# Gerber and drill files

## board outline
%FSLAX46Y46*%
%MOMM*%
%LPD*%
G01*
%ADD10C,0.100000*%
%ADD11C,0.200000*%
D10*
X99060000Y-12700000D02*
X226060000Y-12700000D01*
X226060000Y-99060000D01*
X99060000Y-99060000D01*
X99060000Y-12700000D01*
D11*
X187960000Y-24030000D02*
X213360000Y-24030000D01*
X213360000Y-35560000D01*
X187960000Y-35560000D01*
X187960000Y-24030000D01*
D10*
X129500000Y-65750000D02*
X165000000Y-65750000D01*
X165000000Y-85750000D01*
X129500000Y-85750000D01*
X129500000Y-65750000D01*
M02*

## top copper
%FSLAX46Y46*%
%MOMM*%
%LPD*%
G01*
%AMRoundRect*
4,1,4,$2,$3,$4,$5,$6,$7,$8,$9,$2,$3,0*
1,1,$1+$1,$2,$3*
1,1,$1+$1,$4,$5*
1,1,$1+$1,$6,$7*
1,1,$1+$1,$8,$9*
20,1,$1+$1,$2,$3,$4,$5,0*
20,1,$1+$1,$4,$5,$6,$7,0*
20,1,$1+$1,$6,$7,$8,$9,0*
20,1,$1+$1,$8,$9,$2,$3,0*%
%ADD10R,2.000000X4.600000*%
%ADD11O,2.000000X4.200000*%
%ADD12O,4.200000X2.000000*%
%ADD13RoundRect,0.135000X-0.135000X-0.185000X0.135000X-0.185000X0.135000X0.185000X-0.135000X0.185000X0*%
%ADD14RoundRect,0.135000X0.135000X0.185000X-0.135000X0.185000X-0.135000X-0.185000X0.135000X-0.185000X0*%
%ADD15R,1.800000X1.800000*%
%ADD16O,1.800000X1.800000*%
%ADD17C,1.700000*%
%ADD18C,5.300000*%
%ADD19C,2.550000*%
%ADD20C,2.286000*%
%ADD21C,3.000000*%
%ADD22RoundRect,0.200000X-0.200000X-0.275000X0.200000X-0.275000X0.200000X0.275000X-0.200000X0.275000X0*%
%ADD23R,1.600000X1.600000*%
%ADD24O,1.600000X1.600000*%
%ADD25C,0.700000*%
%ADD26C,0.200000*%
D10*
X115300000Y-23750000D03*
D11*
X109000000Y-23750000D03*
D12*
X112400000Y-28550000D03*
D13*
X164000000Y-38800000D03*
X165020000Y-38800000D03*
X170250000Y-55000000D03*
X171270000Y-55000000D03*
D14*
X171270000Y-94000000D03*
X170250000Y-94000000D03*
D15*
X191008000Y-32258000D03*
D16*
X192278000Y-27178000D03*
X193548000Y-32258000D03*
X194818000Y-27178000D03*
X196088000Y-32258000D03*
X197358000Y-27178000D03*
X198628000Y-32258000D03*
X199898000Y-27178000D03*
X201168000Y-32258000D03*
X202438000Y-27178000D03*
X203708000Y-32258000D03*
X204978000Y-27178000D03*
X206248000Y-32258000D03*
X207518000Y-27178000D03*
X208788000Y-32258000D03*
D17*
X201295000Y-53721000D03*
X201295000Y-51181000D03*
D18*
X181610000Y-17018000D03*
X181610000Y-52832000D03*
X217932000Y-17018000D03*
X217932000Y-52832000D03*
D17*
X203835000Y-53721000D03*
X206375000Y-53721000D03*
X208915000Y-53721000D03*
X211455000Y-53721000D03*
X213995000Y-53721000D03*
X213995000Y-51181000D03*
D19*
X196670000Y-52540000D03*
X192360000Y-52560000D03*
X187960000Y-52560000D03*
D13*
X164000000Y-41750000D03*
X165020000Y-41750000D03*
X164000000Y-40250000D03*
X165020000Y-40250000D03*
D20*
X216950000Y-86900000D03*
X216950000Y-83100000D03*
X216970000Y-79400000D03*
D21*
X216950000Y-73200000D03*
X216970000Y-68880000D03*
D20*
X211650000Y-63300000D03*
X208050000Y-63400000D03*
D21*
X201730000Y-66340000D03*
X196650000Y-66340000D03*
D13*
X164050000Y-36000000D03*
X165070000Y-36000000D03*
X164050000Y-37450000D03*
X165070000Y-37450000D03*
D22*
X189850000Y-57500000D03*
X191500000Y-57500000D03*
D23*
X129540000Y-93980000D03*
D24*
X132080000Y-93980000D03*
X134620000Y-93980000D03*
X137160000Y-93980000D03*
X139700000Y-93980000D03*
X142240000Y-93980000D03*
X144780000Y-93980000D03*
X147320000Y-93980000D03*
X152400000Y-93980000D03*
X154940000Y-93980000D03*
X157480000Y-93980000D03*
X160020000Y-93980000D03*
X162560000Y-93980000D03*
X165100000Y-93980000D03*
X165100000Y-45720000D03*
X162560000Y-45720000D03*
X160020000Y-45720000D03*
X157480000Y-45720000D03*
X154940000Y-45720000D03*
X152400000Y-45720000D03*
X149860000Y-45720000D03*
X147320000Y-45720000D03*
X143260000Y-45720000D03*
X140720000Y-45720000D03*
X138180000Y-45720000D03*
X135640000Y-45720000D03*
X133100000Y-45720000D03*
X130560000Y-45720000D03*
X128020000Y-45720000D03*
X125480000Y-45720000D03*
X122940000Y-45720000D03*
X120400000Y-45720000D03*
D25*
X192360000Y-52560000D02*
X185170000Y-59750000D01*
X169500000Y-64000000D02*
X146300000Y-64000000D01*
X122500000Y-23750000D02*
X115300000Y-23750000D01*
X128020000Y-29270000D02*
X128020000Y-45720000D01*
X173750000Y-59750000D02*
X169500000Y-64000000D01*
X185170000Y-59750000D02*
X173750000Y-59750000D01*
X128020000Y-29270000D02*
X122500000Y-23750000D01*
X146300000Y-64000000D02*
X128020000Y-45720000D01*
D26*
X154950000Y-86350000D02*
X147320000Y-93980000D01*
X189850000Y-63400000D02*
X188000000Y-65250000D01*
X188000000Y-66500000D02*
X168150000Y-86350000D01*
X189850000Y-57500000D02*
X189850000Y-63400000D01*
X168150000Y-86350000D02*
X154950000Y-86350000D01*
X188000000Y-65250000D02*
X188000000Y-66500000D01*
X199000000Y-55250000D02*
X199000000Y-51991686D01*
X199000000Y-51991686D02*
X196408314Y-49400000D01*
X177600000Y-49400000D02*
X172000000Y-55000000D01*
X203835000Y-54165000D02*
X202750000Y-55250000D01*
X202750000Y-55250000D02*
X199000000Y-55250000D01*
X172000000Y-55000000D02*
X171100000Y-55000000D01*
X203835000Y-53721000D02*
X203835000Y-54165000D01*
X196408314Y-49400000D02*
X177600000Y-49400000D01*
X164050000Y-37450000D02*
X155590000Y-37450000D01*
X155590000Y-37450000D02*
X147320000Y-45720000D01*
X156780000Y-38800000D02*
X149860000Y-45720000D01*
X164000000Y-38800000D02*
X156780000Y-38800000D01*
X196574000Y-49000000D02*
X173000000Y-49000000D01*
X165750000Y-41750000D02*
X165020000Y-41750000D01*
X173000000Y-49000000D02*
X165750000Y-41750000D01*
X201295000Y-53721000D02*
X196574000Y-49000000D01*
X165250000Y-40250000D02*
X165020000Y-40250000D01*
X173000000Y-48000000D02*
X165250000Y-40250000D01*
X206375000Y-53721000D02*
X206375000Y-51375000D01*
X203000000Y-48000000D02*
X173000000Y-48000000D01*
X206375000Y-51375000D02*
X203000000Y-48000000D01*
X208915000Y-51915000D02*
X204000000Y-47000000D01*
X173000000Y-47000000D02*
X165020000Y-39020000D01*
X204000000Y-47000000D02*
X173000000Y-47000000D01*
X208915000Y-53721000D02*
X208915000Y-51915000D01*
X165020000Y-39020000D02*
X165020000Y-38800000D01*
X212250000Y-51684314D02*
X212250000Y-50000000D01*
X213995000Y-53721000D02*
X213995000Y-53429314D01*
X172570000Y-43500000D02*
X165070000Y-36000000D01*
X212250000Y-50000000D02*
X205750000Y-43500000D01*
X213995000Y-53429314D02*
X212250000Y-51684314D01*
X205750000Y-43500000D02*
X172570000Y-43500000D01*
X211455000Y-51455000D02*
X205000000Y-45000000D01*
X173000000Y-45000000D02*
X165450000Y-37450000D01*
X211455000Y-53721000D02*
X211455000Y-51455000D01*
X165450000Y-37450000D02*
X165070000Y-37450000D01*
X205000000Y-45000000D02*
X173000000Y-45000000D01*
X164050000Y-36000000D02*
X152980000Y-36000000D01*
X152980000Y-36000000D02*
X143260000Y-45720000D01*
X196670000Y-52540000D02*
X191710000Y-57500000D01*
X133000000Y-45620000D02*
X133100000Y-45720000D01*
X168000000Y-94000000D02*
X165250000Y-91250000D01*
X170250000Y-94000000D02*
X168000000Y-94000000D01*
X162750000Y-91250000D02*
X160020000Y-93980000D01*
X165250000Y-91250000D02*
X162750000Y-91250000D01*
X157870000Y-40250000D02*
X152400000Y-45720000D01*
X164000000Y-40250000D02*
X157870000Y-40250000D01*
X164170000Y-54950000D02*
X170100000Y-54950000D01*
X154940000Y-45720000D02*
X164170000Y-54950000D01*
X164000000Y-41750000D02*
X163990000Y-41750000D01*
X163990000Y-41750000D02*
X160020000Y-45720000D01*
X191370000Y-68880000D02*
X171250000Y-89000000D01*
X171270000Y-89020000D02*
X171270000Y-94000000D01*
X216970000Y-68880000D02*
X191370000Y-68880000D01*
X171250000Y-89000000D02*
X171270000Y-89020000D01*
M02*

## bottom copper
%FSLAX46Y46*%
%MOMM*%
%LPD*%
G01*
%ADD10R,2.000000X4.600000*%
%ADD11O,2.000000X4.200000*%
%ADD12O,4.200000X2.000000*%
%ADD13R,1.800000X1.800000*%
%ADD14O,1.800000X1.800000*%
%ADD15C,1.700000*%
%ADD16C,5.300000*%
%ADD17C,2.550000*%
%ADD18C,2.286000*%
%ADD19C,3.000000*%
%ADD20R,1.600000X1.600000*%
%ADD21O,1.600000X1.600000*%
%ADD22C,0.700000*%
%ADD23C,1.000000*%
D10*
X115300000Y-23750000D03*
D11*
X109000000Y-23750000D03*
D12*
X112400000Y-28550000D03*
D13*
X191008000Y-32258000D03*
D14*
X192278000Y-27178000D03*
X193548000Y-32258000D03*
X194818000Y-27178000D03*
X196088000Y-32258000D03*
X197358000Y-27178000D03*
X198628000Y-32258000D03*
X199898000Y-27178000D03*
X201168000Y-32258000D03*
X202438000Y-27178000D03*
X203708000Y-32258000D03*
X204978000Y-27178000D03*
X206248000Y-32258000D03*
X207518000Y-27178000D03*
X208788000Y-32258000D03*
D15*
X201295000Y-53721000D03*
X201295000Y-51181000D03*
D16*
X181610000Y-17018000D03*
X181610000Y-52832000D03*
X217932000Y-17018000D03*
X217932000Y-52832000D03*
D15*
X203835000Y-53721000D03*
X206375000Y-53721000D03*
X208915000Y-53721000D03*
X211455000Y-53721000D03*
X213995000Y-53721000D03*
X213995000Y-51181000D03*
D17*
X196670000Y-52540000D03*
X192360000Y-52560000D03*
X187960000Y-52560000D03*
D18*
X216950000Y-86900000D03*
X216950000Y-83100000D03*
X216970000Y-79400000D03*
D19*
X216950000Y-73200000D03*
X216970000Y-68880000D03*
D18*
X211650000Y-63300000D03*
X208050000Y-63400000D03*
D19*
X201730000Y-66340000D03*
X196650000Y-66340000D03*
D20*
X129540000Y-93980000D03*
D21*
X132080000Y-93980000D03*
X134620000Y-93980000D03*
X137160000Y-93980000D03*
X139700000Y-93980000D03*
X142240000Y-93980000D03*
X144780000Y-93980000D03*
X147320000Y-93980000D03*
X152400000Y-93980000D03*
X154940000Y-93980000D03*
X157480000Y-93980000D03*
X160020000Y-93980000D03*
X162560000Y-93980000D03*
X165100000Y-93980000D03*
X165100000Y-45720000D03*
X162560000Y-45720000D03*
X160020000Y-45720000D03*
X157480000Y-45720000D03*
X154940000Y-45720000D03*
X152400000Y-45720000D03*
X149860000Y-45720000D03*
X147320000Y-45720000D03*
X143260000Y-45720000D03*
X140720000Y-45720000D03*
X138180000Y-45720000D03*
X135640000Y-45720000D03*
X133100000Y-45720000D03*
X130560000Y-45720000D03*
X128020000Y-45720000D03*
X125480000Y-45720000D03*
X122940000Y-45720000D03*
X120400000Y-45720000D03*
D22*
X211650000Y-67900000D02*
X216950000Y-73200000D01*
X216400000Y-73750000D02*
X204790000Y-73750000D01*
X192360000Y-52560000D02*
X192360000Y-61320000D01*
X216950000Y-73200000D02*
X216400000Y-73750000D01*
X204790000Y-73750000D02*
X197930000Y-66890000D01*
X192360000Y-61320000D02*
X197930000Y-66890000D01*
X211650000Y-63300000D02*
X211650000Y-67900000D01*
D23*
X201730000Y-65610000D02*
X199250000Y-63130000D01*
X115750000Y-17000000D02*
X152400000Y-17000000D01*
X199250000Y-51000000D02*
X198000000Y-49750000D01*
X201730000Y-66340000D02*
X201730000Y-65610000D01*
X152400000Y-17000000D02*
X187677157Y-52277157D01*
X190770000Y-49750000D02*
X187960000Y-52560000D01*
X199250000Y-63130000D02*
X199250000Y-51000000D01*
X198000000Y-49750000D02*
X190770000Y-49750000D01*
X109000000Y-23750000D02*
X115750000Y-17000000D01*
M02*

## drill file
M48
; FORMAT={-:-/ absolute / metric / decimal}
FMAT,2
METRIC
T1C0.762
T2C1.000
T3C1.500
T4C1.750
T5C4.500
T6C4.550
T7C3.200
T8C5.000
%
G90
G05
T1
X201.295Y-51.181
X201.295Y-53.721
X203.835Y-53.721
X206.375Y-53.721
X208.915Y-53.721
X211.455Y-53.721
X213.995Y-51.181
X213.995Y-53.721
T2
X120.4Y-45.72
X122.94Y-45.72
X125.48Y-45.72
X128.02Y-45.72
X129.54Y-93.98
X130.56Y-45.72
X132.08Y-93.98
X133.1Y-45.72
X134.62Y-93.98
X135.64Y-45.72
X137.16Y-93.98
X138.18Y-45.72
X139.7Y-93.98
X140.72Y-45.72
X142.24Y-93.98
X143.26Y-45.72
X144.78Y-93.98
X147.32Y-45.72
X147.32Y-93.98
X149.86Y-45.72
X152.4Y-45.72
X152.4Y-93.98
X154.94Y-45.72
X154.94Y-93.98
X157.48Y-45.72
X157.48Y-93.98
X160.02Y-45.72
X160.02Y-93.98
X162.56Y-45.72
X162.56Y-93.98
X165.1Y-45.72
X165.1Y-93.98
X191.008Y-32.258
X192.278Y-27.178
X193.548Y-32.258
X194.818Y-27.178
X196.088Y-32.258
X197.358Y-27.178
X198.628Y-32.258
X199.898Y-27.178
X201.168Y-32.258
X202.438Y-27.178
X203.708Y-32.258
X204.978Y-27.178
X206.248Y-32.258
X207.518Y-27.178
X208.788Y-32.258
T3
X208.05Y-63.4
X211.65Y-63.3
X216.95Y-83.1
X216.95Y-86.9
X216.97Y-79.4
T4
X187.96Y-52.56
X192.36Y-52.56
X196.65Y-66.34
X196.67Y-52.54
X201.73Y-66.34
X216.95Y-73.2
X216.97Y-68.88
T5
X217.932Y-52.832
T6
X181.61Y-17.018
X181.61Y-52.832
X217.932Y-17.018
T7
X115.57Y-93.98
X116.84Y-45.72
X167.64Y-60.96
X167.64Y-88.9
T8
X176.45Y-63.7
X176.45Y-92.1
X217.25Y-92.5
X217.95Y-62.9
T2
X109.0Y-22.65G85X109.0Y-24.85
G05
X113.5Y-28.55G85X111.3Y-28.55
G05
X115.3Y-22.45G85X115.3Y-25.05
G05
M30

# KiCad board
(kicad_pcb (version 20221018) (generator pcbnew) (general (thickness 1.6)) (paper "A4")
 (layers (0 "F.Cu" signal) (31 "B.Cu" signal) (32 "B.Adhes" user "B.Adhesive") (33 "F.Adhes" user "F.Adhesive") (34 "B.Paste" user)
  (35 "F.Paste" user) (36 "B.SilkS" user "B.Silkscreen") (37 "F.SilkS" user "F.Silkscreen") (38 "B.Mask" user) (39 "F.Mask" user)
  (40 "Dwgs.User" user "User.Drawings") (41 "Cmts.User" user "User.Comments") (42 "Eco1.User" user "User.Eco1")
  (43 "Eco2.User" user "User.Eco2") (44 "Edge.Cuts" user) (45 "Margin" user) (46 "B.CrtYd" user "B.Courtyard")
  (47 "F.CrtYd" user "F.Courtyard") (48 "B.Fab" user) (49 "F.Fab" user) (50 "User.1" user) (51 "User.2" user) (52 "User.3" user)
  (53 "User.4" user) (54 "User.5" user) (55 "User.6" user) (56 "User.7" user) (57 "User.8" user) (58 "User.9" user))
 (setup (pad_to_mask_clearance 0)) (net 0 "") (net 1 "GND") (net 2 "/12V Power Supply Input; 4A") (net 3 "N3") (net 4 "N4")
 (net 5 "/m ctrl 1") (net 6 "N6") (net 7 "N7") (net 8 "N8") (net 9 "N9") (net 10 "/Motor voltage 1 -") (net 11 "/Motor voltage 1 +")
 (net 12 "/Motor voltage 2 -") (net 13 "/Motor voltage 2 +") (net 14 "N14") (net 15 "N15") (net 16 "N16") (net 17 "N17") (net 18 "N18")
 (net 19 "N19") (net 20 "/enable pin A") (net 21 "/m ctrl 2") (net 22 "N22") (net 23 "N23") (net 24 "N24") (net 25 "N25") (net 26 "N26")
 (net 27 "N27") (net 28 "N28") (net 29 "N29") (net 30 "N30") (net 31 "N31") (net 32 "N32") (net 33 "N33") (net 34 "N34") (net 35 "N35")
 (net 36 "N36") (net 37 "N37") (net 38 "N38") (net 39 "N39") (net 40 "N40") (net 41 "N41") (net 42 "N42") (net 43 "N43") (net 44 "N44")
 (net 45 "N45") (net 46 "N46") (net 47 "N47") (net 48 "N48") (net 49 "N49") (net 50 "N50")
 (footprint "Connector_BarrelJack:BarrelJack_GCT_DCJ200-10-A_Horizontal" (layer "F.Cu") (at 115.3 23.75 -90)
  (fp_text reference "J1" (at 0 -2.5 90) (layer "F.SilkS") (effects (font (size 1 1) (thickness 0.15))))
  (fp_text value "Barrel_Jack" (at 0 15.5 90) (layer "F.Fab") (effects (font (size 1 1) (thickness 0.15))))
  (pad "1" thru_hole rect (at 0 0 270) (size 4.6 2) (drill oval 3.6 1) (layers "*.Cu" "*.Mask") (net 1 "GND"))
  (pad "2" thru_hole oval (at 0 6.3 270) (size 4.2 2) (drill oval 3.2 1) (layers "*.Cu" "*.Mask") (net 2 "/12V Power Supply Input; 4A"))
  (pad "3" thru_hole oval (at 4.8 2.9 270) (size 2 4.2) (drill oval 1 3.2) (layers "*.Cu" "*.Mask")))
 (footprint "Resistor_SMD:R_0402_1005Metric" (layer "F.Cu") (at 164.51 38.8)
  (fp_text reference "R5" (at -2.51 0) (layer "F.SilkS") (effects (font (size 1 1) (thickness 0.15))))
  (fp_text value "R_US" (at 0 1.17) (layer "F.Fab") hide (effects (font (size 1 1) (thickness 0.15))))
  (pad "1" smd roundrect (at -0.51 0) (size 0.54 0.64) (layers "F.Cu" "F.Paste" "F.Mask") (roundrect_rratio 0.25) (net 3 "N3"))
  (pad "2" smd roundrect (at 0.51 0) (size 0.54 0.64) (layers "F.Cu" "F.Paste" "F.Mask") (roundrect_rratio 0.25) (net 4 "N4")))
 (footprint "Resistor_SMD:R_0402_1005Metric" (layer "F.Cu") (at 170.76 55)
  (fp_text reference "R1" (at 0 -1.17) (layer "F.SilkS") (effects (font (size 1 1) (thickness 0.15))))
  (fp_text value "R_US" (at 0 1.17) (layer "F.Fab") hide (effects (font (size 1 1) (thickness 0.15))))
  (pad "1" smd roundrect (at -0.51 0) (size 0.54 0.64) (layers "F.Cu" "F.Paste" "F.Mask") (roundrect_rratio 0.25) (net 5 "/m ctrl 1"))
  (pad "2" smd roundrect (at 0.51 0) (size 0.54 0.64) (layers "F.Cu" "F.Paste" "F.Mask") (roundrect_rratio 0.25) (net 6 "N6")))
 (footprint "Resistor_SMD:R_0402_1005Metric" (layer "F.Cu") (at 170.76 94 180)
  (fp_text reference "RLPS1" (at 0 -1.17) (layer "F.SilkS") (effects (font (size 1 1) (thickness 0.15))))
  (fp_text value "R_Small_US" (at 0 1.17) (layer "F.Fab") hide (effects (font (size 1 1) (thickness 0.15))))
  (pad "1" smd roundrect (at -0.51 0 180) (size 0.54 0.64) (layers "F.Cu" "F.Paste" "F.Mask") (roundrect_rratio 0.25) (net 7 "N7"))
  (pad "2" smd roundrect (at 0.51 0 180) (size 0.54 0.64) (layers "F.Cu" "F.Paste" "F.Mask") (roundrect_rratio 0.25) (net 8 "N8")))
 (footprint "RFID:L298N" (layer "F.Cu") (at 200.66 35.56)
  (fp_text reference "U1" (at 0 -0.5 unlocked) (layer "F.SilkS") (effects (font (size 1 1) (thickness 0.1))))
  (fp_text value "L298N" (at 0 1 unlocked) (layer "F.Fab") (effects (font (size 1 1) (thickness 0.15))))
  (pad "1" thru_hole rect (at -9.652 -3.302) (size 1.8 1.8) (drill 1) (layers "*.Cu" "*.Mask") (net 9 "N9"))
  (pad "2" thru_hole oval (at -8.382 -8.382) (size 1.8 1.8) (drill 1) (layers "*.Cu" "*.Mask") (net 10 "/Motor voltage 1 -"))
  (pad "3" thru_hole oval (at -7.112 -3.302) (size 1.8 1.8) (drill 1) (layers "*.Cu" "*.Mask") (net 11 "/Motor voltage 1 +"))
  (pad "4" thru_hole oval (at -5.842 -8.382) (size 1.8 1.8) (drill 1) (layers "*.Cu" "*.Mask"))
  (pad "5" thru_hole oval (at -4.572 -3.302) (size 1.8 1.8) (drill 1) (layers "*.Cu" "*.Mask"))
  (pad "6" thru_hole oval (at -3.302 -8.382) (size 1.8 1.8) (drill 1) (layers "*.Cu" "*.Mask"))
  (pad "7" thru_hole oval (at -2.032 -3.302) (size 1.8 1.8) (drill 1) (layers "*.Cu" "*.Mask"))
  (pad "8" thru_hole oval (at -0.762 -8.382) (size 1.8 1.8) (drill 1) (layers "*.Cu" "*.Mask"))
  (pad "9" thru_hole oval (at 0.508 -3.302) (size 1.8 1.8) (drill 1) (layers "*.Cu" "*.Mask"))
  (pad "10" thru_hole oval (at 1.778 -8.382) (size 1.8 1.8) (drill 1) (layers "*.Cu" "*.Mask"))
  (pad "11" thru_hole oval (at 3.048 -3.302) (size 1.8 1.8) (drill 1) (layers "*.Cu" "*.Mask"))
  (pad "12" thru_hole oval (at 4.318 -8.382) (size 1.8 1.8) (drill 1) (layers "*.Cu" "*.Mask"))
  (pad "13" thru_hole oval (at 5.588 -3.302) (size 1.8 1.8) (drill 1) (layers "*.Cu" "*.Mask") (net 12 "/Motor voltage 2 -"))
  (pad "14" thru_hole oval (at 6.858 -8.382) (size 1.8 1.8) (drill 1) (layers "*.Cu" "*.Mask") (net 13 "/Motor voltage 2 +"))
  (pad "15" thru_hole oval (at 8.128 -3.302) (size 1.8 1.8) (drill 1) (layers "*.Cu" "*.Mask") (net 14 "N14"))
  (pad "23" thru_hole circle (at 0.635 18.161) (size 1.7 1.7) (drill 0.762) (layers "*.Cu" "*.Mask") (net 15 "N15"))
  (pad "24" thru_hole circle (at 0.635 15.621) (size 1.7 1.7) (drill 0.762) (layers "*.Cu" "*.Mask"))
  (pad "25" thru_hole circle (at -19.05 -18.542) (size 5.3 5.3) (drill 4.55) (layers "*.Cu" "*.Mask"))
  (pad "25" thru_hole circle (at -19.05 17.272) (size 5.3 5.3) (drill 4.55) (layers "*.Cu" "*.Mask"))
  (pad "25" thru_hole circle (at 17.272 -18.542) (size 5.3 5.3) (drill 4.55) (layers "*.Cu" "*.Mask"))
  (pad "25" thru_hole circle (at 17.272 17.272) (size 5.3 5.3) (drill 4.5) (layers "*.Cu" "*.Mask"))
  (pad "26" thru_hole circle (at 3.175 18.161) (size 1.7 1.7) (drill 0.762) (layers "*.Cu" "*.Mask") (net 6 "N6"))
  (pad "27" thru_hole circle (at 5.715 18.161) (size 1.7 1.7) (drill 0.762) (layers "*.Cu" "*.Mask") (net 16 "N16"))
  (pad "28" thru_hole circle (at 8.255 18.161) (size 1.7 1.7) (drill 0.762) (layers "*.Cu" "*.Mask") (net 4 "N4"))
  (pad "29" thru_hole circle (at 10.795 18.161) (size 1.7 1.7) (drill 0.762) (layers "*.Cu" "*.Mask") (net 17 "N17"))
  (pad "30" thru_hole circle (at 13.335 18.161) (size 1.7 1.7) (drill 0.762) (layers "*.Cu" "*.Mask") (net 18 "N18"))
  (pad "31" thru_hole circle (at 13.335 15.621) (size 1.7 1.7) (drill 0.762) (layers "*.Cu" "*.Mask"))
  (pad "32" thru_hole circle (at -3.99 16.98) (size 2.55 2.55) (drill 1.75) (layers "*.Cu" "*.Mask") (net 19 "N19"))
  (pad "33" thru_hole circle (at -8.3 17) (size 2.55 2.55) (drill 1.75) (layers "*.Cu" "*.Mask") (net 1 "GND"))
  (pad "34" thru_hole circle (at -12.7 17) (size 2.55 2.55) (drill 1.75) (layers "*.Cu" "*.Mask") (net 2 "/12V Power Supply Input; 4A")))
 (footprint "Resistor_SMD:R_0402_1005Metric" (layer "F.Cu") (at 164.51 41.75)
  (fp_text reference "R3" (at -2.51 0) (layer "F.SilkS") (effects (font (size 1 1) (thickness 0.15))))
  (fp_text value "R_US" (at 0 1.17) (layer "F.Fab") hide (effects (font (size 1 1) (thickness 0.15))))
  (pad "1" smd roundrect (at -0.51 0) (size 0.54 0.64) (layers "F.Cu" "F.Paste" "F.Mask") (roundrect_rratio 0.25) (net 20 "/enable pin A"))
  (pad "2" smd roundrect (at 0.51 0) (size 0.54 0.64) (layers "F.Cu" "F.Paste" "F.Mask") (roundrect_rratio 0.25) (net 15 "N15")))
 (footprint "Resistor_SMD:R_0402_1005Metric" (layer "F.Cu") (at 164.51 40.25)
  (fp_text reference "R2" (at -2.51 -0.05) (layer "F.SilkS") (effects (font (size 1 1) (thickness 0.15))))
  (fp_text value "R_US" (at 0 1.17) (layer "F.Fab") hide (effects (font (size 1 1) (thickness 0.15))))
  (pad "1" smd roundrect (at -0.51 0) (size 0.54 0.64) (layers "F.Cu" "F.Paste" "F.Mask") (roundrect_rratio 0.25) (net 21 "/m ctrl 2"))
  (pad "2" smd roundrect (at 0.51 0) (size 0.54 0.64) (layers "F.Cu" "F.Paste" "F.Mask") (roundrect_rratio 0.25) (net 16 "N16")))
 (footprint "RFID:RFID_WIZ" (layer "F.Cu") (at 196.65 76.5)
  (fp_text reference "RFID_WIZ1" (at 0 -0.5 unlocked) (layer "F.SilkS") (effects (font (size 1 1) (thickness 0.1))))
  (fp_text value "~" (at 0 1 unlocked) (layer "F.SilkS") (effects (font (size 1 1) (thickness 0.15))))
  (pad "" np_thru_hole circle (at -20.2 -12.8) (size 5 5) (drill 5) (layers "F&B.Cu" "*.Mask"))
  (pad "" np_thru_hole circle (at -20.2 15.6) (size 5 5) (drill 5) (layers "F&B.Cu" "*.Mask"))
  (pad "" np_thru_hole circle (at 20.6 16) (size 5 5) (drill 5) (layers "F&B.Cu" "*.Mask"))
  (pad "" np_thru_hole circle (at 21.3 -13.6) (size 5 5) (drill 5) (layers "F&B.Cu" "*.Mask"))
  (pad "1" thru_hole circle (at 20.3 10.4) (size 2.286 2.286) (drill 1.5) (layers "*.Cu" "*.Mask") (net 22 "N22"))
  (pad "2" thru_hole circle (at 20.3 6.6) (size 2.286 2.286) (drill 1.5) (layers "*.Cu" "*.Mask") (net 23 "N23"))
  (pad "3" thru_hole circle (at 20.32 2.9) (size 2.286 2.286) (drill 1.5) (layers "*.Cu" "*.Mask") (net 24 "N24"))
  (pad "4" thru_hole circle (at 20.3 -3.3) (size 3 3) (drill 1.75) (layers "*.Cu" "*.Mask") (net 1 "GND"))
  (pad "5" thru_hole circle (at 20.32 -7.62) (size 3 3) (drill 1.75) (layers "*.Cu" "*.Mask") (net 7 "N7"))
  (pad "6" thru_hole circle (at 15 -13.2) (size 2.286 2.286) (drill 1.5) (layers "*.Cu" "*.Mask") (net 1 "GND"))
  (pad "7" thru_hole circle (at 11.4 -13.1) (size 2.286 2.286) (drill 1.5) (layers "*.Cu" "*.Mask"))
  (pad "8" thru_hole circle (at 5.08 -10.16) (size 3 3) (drill 1.75) (layers "*.Cu" "*.Mask") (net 2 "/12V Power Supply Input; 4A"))
  (pad "9" thru_hole circle (at 0 -10.16) (size 3 3) (drill 1.75) (layers "*.Cu" "*.Mask") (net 1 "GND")))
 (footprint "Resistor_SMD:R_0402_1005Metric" (layer "F.Cu") (at 164.56 36)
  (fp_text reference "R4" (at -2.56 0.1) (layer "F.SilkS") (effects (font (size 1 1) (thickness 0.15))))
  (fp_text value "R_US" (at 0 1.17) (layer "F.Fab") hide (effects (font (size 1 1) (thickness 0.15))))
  (pad "1" smd roundrect (at -0.51 0) (size 0.54 0.64) (layers "F.Cu" "F.Paste" "F.Mask") (roundrect_rratio 0.25) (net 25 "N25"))
  (pad "2" smd roundrect (at 0.51 0) (size 0.54 0.64) (layers "F.Cu" "F.Paste" "F.Mask") (roundrect_rratio 0.25) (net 18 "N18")))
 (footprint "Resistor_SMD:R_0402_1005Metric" (layer "F.Cu") (at 164.56 37.45)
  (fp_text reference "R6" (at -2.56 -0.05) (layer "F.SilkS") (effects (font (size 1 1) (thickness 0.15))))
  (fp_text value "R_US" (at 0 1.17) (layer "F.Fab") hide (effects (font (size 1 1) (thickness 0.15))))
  (pad "1" smd roundrect (at -0.51 0) (size 0.54 0.64) (layers "F.Cu" "F.Paste" "F.Mask") (roundrect_rratio 0.25) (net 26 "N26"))
  (pad "2" smd roundrect (at 0.51 0) (size 0.54 0.64) (layers "F.Cu" "F.Paste" "F.Mask") (roundrect_rratio 0.25) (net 17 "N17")))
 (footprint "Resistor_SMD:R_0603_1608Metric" (layer "F.Cu") (at 190.675 57.5)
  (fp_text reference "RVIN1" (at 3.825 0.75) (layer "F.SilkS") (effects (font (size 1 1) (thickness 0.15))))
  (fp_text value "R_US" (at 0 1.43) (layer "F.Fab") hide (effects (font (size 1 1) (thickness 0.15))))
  (pad "1" smd roundrect (at -0.825 0) (size 0.8 0.95) (layers "F.Cu" "F.Paste" "F.Mask") (roundrect_rratio 0.25) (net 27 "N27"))
  (pad "2" smd roundrect (at 0.825 0) (size 0.8 0.95) (layers "F.Cu" "F.Paste" "F.Mask") (roundrect_rratio 0.25) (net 19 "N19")))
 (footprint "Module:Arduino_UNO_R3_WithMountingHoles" (layer "B.Cu") (at 129.54 93.98)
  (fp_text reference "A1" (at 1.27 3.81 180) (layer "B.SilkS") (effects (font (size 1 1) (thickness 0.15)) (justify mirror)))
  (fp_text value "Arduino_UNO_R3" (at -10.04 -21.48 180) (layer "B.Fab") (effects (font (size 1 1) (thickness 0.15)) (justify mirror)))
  (pad "" np_thru_hole circle (at -13.97 0 270) (size 3.2 3.2) (drill 3.2) (layers "*.Cu" "*.Mask"))
  (pad "" np_thru_hole circle (at -12.7 -48.26 270) (size 3.2 3.2) (drill 3.2) (layers "*.Cu" "*.Mask"))
  (pad "" np_thru_hole circle (at 38.1 -33.02 270) (size 3.2 3.2) (drill 3.2) (layers "*.Cu" "*.Mask"))
  (pad "" np_thru_hole circle (at 38.1 -5.08 270) (size 3.2 3.2) (drill 3.2) (layers "*.Cu" "*.Mask"))
  (pad "1" thru_hole rect (at 0 0 270) (size 1.6 1.6) (drill 1) (layers "*.Cu" "*.Mask") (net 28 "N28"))
  (pad "2" thru_hole oval (at 2.54 0 270) (size 1.6 1.6) (drill 1) (layers "*.Cu" "*.Mask") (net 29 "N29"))
  (pad "3" thru_hole oval (at 5.08 0 270) (size 1.6 1.6) (drill 1) (layers "*.Cu" "*.Mask") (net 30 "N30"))
  (pad "4" thru_hole oval (at 7.62 0 270) (size 1.6 1.6) (drill 1) (layers "*.Cu" "*.Mask") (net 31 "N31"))
  (pad "5" thru_hole oval (at 10.16 0 270) (size 1.6 1.6) (drill 1) (layers "*.Cu" "*.Mask") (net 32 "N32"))
  (pad "6" thru_hole oval (at 12.7 0 270) (size 1.6 1.6) (drill 1) (layers "*.Cu" "*.Mask") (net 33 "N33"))
  (pad "7" thru_hole oval (at 15.24 0 270) (size 1.6 1.6) (drill 1) (layers "*.Cu" "*.Mask") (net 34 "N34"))
  (pad "8" thru_hole oval (at 17.78 0 270) (size 1.6 1.6) (drill 1) (layers "*.Cu" "*.Mask") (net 27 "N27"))
  (pad "9" thru_hole oval (at 22.86 0 270) (size 1.6 1.6) (drill 1) (layers "*.Cu" "*.Mask") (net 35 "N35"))
  (pad "10" thru_hole oval (at 25.4 0 270) (size 1.6 1.6) (drill 1) (layers "*.Cu" "*.Mask") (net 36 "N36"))
  (pad "11" thru_hole oval (at 27.94 0 270) (size 1.6 1.6) (drill 1) (layers "*.Cu" "*.Mask") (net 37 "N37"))
  (pad "12" thru_hole oval (at 30.48 0 270) (size 1.6 1.6) (drill 1) (layers "*.Cu" "*.Mask") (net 8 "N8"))
  (pad "13" thru_hole oval (at 33.02 0 270) (size 1.6 1.6) (drill 1) (layers "*.Cu" "*.Mask") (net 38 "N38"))
  (pad "14" thru_hole oval (at 35.56 0 270) (size 1.6 1.6) (drill 1) (layers "*.Cu" "*.Mask") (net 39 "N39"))
  (pad "15" thru_hole oval (at 35.56 -48.26 270) (size 1.6 1.6) (drill 1) (layers "*.Cu" "*.Mask") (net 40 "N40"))
  (pad "16" thru_hole oval (at 33.02 -48.26 270) (size 1.6 1.6) (drill 1) (layers "*.Cu" "*.Mask") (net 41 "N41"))
  (pad "17" thru_hole oval (at 30.48 -48.26 270) (size 1.6 1.6) (drill 1) (layers "*.Cu" "*.Mask") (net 20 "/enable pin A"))
  (pad "18" thru_hole oval (at 27.94 -48.26 270) (size 1.6 1.6) (drill 1) (layers "*.Cu" "*.Mask") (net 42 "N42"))
  (pad "19" thru_hole oval (at 25.4 -48.26 270) (size 1.6 1.6) (drill 1) (layers "*.Cu" "*.Mask") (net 5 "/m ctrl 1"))
  (pad "20" thru_hole oval (at 22.86 -48.26 270) (size 1.6 1.6) (drill 1) (layers "*.Cu" "*.Mask") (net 21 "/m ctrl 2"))
  (pad "21" thru_hole oval (at 20.32 -48.26 270) (size 1.6 1.6) (drill 1) (layers "*.Cu" "*.Mask") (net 3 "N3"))
  (pad "22" thru_hole oval (at 17.78 -48.26 270) (size 1.6 1.6) (drill 1) (layers "*.Cu" "*.Mask") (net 26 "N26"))
  (pad "23" thru_hole oval (at 13.72 -48.26 270) (size 1.6 1.6) (drill 1) (layers "*.Cu" "*.Mask") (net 25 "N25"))
  (pad "24" thru_hole oval (at 11.18 -48.26 270) (size 1.6 1.6) (drill 1) (layers "*.Cu" "*.Mask") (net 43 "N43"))
  (pad "25" thru_hole oval (at 8.64 -48.26 270) (size 1.6 1.6) (drill 1) (layers "*.Cu" "*.Mask") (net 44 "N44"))
  (pad "26" thru_hole oval (at 6.1 -48.26 270) (size 1.6 1.6) (drill 1) (layers "*.Cu" "*.Mask") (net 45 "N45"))
  (pad "27" thru_hole oval (at 3.56 -48.26 270) (size 1.6 1.6) (drill 1) (layers "*.Cu" "*.Mask") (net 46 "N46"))
  (pad "28" thru_hole oval (at 1.02 -48.26 270) (size 1.6 1.6) (drill 1) (layers "*.Cu" "*.Mask") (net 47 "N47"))
  (pad "29" thru_hole oval (at -1.52 -48.26 270) (size 1.6 1.6) (drill 1) (layers "*.Cu" "*.Mask") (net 1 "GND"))
  (pad "30" thru_hole oval (at -4.06 -48.26 270) (size 1.6 1.6) (drill 1) (layers "*.Cu" "*.Mask") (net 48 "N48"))
  (pad "31" thru_hole oval (at -6.6 -48.26 270) (size 1.6 1.6) (drill 1) (layers "*.Cu" "*.Mask") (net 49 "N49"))
  (pad "32" thru_hole oval (at -9.14 -48.26 270) (size 1.6 1.6) (drill 1) (layers "*.Cu" "*.Mask") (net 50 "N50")))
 (gr_rect (start 99.06 12.7) (end 226.06 99.06) (stroke (width 0.1) (type default)) (fill none) (layer "Edge.Cuts"))
 (gr_rect (start 187.96 24.03) (end 213.36 35.56) (stroke (width 0.2) (type default)) (fill none) (layer "Edge.Cuts"))
 (gr_rect (start 129.5 65.75) (end 165 85.75) (stroke (width 0.1) (type default)) (fill none) (layer "Edge.Cuts"))
 (segment (start 192.36 52.56) (end 185.17 59.75) (width 0.7) (layer "F.Cu") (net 1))
 (segment (start 169.5 64) (end 146.3 64) (width 0.7) (layer "F.Cu") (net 1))
 (segment (start 122.5 23.75) (end 115.3 23.75) (width 0.7) (layer "F.Cu") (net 1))
 (segment (start 128.02 29.27) (end 128.02 45.72) (width 0.7) (layer "F.Cu") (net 1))
 (segment (start 173.75 59.75) (end 169.5 64) (width 0.7) (layer "F.Cu") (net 1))
 (segment (start 185.17 59.75) (end 173.75 59.75) (width 0.7) (layer "F.Cu") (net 1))
 (segment (start 128.02 29.27) (end 122.5 23.75) (width 0.7) (layer "F.Cu") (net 1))
 (segment (start 146.3 64) (end 128.02 45.72) (width 0.7) (layer "F.Cu") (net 1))
 (segment (start 211.65 67.9) (end 216.95 73.2) (width 0.7) (layer "B.Cu") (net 1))
 (segment (start 216.4 73.75) (end 204.79 73.75) (width 0.7) (layer "B.Cu") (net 1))
 (segment (start 192.36 52.56) (end 192.36 61.32) (width 0.7) (layer "B.Cu") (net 1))
 (segment (start 216.95 73.2) (end 216.4 73.75) (width 0.7) (layer "B.Cu") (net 1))
 (segment (start 204.79 73.75) (end 197.93 66.89) (width 0.7) (layer "B.Cu") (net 1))
 (segment (start 192.36 61.32) (end 197.93 66.89) (width 0.7) (layer "B.Cu") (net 1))
 (segment (start 211.65 63.3) (end 211.65 67.9) (width 0.7) (layer "B.Cu") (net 1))
 (segment (start 154.95 86.35) (end 147.32 93.98) (width 0.2) (layer "F.Cu") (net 27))
 (segment (start 189.85 63.4) (end 188 65.25) (width 0.2) (layer "F.Cu") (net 27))
 (segment (start 188 66.5) (end 168.15 86.35) (width 0.2) (layer "F.Cu") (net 27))
 (segment (start 189.85 57.5) (end 189.85 63.4) (width 0.2) (layer "F.Cu") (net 27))
 (segment (start 168.15 86.35) (end 154.95 86.35) (width 0.2) (layer "F.Cu") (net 27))
 (segment (start 188 65.25) (end 188 66.5) (width 0.2) (layer "F.Cu") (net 27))
 (segment (start 199 55.25) (end 199 51.991686) (width 0.2) (layer "F.Cu") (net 6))
 (segment (start 199 51.991686) (end 196.408314 49.4) (width 0.2) (layer "F.Cu") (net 6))
 (segment (start 177.6 49.4) (end 172 55) (width 0.2) (layer "F.Cu") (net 6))
 (segment (start 203.835 54.165) (end 202.75 55.25) (width 0.2) (layer "F.Cu") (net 6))
 (segment (start 202.75 55.25) (end 199 55.25) (width 0.2) (layer "F.Cu") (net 6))
 (segment (start 172 55) (end 171.1 55) (width 0.2) (layer "F.Cu") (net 6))
 (segment (start 203.835 53.721) (end 203.835 54.165) (width 0.2) (layer "F.Cu") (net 6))
 (segment (start 196.408314 49.4) (end 177.6 49.4) (width 0.2) (layer "F.Cu") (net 6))
 (segment (start 164.05 37.45) (end 155.59 37.45) (width 0.2) (layer "F.Cu") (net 26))
 (segment (start 155.59 37.45) (end 147.32 45.72) (width 0.2) (layer "F.Cu") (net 26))
 (segment (start 156.78 38.8) (end 149.86 45.72) (width 0.2) (layer "F.Cu") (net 3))
 (segment (start 164 38.8) (end 156.78 38.8) (width 0.2) (layer "F.Cu") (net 3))
 (segment (start 196.574 49) (end 173 49) (width 0.2) (layer "F.Cu") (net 15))
 (segment (start 165.75 41.75) (end 165.02 41.75) (width 0.2) (layer "F.Cu") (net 15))
 (segment (start 173 49) (end 165.75 41.75) (width 0.2) (layer "F.Cu") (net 15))
 (segment (start 201.295 53.721) (end 196.574 49) (width 0.2) (layer "F.Cu") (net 15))
 (segment (start 165.25 40.25) (end 165.02 40.25) (width 0.2) (layer "F.Cu") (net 16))
 (segment (start 173 48) (end 165.25 40.25) (width 0.2) (layer "F.Cu") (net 16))
 (segment (start 206.375 53.721) (end 206.375 51.375) (width 0.2) (layer "F.Cu") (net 16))
 (segment (start 203 48) (end 173 48) (width 0.2) (layer "F.Cu") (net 16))
 (segment (start 206.375 51.375) (end 203 48) (width 0.2) (layer "F.Cu") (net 16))
 (segment (start 208.915 51.915) (end 204 47) (width 0.2) (layer "F.Cu") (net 4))
 (segment (start 173 47) (end 165.02 39.02) (width 0.2) (layer "F.Cu") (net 4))
 (segment (start 204 47) (end 173 47) (width 0.2) (layer "F.Cu") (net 4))
 (segment (start 208.915 53.721) (end 208.915 51.915) (width 0.2) (layer "F.Cu") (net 4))
 (segment (start 165.02 39.02) (end 165.02 38.8) (width 0.2) (layer "F.Cu") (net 4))
 (segment (start 212.25 51.684314) (end 212.25 50) (width 0.2) (layer "F.Cu") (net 18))
 (segment (start 213.995 53.721) (end 213.995 53.429314) (width 0.2) (layer "F.Cu") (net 18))
 (segment (start 172.57 43.5) (end 165.07 36) (width 0.2) (layer "F.Cu") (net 18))
 (segment (start 212.25 50) (end 205.75 43.5) (width 0.2) (layer "F.Cu") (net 18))
 (segment (start 213.995 53.429314) (end 212.25 51.684314) (width 0.2) (layer "F.Cu") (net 18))
 (segment (start 205.75 43.5) (end 172.57 43.5) (width 0.2) (layer "F.Cu") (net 18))
 (segment (start 211.455 51.455) (end 205 45) (width 0.2) (layer "F.Cu") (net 17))
 (segment (start 173 45) (end 165.45 37.45) (width 0.2) (layer "F.Cu") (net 17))
 (segment (start 211.455 53.721) (end 211.455 51.455) (width 0.2) (layer "F.Cu") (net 17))
 (segment (start 165.45 37.45) (end 165.07 37.45) (width 0.2) (layer "F.Cu") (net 17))
 (segment (start 205 45) (end 173 45) (width 0.2) (layer "F.Cu") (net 17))
 (segment (start 164.05 36) (end 152.98 36) (width 0.2) (layer "F.Cu") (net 25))
 (segment (start 152.98 36) (end 143.26 45.72) (width 0.2) (layer "F.Cu") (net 25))
 (segment (start 196.67 52.54) (end 191.71 57.5) (width 0.2) (layer "F.Cu") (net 19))
 (segment (start 133 45.62) (end 133.1 45.72) (width 0.2) (layer "F.Cu") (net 46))
 (segment (start 168 94) (end 165.25 91.25) (width 0.2) (layer "F.Cu") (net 8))
 (segment (start 170.25 94) (end 168 94) (width 0.2) (layer "F.Cu") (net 8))
 (segment (start 162.75 91.25) (end 160.02 93.98) (width 0.2) (layer "F.Cu") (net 8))
 (segment (start 165.25 91.25) (end 162.75 91.25) (width 0.2) (layer "F.Cu") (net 8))
 (segment (start 201.73 65.61) (end 199.25 63.13) (width 1) (layer "B.Cu") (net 2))
 (segment (start 115.75 17) (end 152.4 17) (width 1) (layer "B.Cu") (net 2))
 (segment (start 199.25 51) (end 198 49.75) (width 1) (layer "B.Cu") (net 2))
 (segment (start 201.73 66.34) (end 201.73 65.61) (width 1) (layer "B.Cu") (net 2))
 (segment (start 152.4 17) (end 187.677157 52.277157) (width 1) (layer "B.Cu") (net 2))
 (segment (start 190.77 49.75) (end 187.96 52.56) (width 1) (layer "B.Cu") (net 2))
 (segment (start 199.25 63.13) (end 199.25 51) (width 1) (layer "B.Cu") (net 2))
 (segment (start 198 49.75) (end 190.77 49.75) (width 1) (layer "B.Cu") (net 2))
 (segment (start 109 23.75) (end 115.75 17) (width 1) (layer "B.Cu") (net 2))
 (segment (start 157.87 40.25) (end 152.4 45.72) (width 0.2) (layer "F.Cu") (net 21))
 (segment (start 164 40.25) (end 157.87 40.25) (width 0.2) (layer "F.Cu") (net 21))
 (segment (start 164.17 54.95) (end 170.1 54.95) (width 0.2) (layer "F.Cu") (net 5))
 (segment (start 154.94 45.72) (end 164.17 54.95) (width 0.2) (layer "F.Cu") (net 5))
 (segment (start 164 41.75) (end 163.99 41.75) (width 0.2) (layer "F.Cu") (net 20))
 (segment (start 163.99 41.75) (end 160.02 45.72) (width 0.2) (layer "F.Cu") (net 20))
 (segment (start 191.37 68.88) (end 171.25 89) (width 0.2) (layer "F.Cu") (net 7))
 (segment (start 171.27 89.02) (end 171.27 94) (width 0.2) (layer "F.Cu") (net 7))
 (segment (start 216.97 68.88) (end 191.37 68.88) (width 0.2) (layer "F.Cu") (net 7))
 (segment (start 171.25 89) (end 171.27 89.02) (width 0.2) (layer "F.Cu") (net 7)))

